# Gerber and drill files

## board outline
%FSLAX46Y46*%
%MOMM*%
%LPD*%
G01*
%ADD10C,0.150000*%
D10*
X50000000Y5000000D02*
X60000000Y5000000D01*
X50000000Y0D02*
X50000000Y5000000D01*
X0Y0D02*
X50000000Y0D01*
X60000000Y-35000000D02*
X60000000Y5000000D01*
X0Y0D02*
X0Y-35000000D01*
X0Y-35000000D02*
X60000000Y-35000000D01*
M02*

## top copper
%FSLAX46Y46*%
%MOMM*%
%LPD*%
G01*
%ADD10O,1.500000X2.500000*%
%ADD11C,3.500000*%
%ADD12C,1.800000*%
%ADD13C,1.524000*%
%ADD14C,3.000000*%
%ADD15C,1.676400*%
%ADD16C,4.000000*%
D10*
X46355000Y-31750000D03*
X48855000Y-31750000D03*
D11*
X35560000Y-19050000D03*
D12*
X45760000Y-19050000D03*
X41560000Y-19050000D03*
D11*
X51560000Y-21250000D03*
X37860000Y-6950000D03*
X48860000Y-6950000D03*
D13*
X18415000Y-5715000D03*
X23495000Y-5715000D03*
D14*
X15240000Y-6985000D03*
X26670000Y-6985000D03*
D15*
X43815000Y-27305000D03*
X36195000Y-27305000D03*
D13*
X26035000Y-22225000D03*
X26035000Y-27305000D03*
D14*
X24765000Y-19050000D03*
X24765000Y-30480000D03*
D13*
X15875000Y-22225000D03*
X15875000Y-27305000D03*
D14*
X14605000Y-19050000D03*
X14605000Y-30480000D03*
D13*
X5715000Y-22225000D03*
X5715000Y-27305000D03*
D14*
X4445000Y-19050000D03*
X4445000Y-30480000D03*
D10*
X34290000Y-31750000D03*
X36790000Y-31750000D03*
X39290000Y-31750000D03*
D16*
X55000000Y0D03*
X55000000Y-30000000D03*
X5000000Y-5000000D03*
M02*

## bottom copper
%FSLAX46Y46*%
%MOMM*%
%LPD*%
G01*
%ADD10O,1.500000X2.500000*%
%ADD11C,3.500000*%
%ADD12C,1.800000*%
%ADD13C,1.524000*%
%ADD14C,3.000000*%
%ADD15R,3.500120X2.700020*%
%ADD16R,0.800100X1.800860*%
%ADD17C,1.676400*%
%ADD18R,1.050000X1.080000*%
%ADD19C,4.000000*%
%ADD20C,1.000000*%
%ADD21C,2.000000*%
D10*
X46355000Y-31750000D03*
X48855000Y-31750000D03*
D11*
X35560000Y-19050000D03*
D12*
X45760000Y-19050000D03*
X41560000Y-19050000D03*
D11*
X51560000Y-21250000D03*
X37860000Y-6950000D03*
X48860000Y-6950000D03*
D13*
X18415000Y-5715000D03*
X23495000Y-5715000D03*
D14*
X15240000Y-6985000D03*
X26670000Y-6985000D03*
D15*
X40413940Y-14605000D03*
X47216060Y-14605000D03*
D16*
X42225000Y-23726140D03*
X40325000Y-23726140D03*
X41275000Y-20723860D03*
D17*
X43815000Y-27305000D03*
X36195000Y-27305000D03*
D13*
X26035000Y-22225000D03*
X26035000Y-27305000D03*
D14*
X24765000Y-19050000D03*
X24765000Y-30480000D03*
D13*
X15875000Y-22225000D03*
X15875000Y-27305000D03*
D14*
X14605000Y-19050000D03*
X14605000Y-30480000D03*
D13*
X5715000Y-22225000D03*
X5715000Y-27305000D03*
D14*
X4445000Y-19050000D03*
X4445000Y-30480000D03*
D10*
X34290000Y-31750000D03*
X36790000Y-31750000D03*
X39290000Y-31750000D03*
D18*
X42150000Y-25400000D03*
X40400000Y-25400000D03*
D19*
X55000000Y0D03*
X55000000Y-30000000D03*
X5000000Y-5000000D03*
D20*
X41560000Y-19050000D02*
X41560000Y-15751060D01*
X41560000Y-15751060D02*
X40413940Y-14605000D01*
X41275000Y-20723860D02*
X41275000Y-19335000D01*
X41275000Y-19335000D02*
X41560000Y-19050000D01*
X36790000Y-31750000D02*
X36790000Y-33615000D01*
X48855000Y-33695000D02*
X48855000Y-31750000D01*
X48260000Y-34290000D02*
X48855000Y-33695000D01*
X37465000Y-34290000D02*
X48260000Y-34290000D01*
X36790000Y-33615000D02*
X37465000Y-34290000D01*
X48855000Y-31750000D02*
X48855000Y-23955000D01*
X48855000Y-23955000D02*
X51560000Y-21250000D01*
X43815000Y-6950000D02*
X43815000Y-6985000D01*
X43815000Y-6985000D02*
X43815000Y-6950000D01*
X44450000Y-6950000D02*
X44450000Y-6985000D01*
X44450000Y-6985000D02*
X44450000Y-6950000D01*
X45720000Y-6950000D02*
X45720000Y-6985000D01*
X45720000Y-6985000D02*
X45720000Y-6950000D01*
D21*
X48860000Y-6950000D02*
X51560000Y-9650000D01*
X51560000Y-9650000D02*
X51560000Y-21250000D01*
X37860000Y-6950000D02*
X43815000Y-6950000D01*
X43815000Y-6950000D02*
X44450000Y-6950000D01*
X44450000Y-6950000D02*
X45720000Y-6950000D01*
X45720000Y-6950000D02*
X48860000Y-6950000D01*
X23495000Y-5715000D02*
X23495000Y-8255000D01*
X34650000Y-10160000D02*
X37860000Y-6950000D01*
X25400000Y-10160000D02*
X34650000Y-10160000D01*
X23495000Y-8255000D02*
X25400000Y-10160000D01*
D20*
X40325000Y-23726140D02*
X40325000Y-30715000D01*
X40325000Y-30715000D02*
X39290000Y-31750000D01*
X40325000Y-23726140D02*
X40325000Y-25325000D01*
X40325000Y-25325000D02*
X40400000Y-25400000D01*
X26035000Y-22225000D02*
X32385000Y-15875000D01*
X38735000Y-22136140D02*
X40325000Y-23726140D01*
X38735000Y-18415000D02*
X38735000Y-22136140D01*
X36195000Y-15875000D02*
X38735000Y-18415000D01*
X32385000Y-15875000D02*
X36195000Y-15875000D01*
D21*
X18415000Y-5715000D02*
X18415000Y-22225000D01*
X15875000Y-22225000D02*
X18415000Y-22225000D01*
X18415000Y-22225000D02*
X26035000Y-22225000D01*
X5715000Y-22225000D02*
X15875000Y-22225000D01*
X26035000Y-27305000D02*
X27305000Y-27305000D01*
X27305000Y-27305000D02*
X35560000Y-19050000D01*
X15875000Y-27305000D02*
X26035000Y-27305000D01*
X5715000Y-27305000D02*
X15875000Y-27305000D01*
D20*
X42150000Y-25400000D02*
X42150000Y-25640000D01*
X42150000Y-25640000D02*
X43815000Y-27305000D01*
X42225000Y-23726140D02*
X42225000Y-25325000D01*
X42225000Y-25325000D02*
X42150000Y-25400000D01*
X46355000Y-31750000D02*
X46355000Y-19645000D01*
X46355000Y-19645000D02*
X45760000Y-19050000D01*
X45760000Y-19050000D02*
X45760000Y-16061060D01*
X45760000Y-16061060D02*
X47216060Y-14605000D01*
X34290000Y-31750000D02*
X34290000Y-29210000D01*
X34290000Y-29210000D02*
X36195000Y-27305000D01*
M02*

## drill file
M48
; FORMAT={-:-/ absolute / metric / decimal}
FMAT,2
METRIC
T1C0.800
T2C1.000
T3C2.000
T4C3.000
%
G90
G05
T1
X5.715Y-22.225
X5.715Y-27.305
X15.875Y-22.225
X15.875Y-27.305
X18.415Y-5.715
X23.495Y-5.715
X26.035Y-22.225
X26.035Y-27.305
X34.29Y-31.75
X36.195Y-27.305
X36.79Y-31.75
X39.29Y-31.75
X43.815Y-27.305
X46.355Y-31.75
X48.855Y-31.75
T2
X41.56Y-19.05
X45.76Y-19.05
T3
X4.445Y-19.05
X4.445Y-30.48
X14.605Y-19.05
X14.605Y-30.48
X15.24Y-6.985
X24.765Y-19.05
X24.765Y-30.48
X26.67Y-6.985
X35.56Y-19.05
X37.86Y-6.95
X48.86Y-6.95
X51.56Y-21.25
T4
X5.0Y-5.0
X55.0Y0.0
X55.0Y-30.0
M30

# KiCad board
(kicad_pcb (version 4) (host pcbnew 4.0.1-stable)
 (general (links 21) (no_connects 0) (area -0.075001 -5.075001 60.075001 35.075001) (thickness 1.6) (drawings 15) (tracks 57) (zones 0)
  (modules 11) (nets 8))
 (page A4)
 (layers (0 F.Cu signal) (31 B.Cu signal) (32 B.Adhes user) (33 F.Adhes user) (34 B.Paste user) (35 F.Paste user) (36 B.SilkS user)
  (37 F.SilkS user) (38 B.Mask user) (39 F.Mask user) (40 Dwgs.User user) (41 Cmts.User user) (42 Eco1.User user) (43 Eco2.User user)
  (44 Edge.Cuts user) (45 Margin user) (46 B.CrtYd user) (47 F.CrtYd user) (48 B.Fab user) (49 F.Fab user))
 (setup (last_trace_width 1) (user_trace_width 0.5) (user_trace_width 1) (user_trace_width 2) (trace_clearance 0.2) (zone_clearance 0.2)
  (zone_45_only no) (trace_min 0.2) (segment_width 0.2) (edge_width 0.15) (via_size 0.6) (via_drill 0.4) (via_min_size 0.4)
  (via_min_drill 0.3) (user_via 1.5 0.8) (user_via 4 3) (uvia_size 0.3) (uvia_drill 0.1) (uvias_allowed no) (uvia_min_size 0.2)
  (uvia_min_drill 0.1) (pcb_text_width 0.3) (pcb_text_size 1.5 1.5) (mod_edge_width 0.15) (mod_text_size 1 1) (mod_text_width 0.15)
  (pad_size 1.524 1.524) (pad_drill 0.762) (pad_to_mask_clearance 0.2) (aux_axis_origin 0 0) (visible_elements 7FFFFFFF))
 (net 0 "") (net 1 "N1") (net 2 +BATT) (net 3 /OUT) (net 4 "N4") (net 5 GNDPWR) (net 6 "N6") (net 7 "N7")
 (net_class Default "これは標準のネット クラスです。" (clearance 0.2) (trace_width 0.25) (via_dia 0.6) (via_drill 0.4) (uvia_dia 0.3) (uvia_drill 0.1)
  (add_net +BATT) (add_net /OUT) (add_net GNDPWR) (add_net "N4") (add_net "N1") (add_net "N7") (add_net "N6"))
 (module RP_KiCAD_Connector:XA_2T (layer F.Cu) (at 46.355 31.75)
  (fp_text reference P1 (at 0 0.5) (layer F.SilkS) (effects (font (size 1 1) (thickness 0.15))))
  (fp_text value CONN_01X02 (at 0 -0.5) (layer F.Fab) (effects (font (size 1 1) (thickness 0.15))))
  (pad 2 thru_hole oval (at 0 0) (size 1.5 2.5) (drill 0.8) (layers *.Cu *.Mask F.SilkS) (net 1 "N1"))
  (pad 1 thru_hole oval (at 2.5 0) (size 1.5 2.5) (drill 0.8) (layers *.Cu *.Mask F.SilkS) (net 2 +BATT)))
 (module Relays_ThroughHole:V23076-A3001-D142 (layer F.Cu) (at 35.56 19.05 180)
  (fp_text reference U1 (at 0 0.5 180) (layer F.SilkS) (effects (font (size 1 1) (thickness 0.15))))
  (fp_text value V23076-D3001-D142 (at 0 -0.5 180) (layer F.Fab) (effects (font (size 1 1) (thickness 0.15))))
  (pad 5 thru_hole circle (at 0 0 180) (size 3.5 3.5) (drill 2) (layers *.Cu *.Mask F.SilkS) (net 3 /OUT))
  (pad 2 thru_hole circle (at -10.2 0 180) (size 1.8 1.8) (drill 1) (layers *.Cu *.Mask F.SilkS) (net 1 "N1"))
  (pad 1 thru_hole circle (at -6 0 180) (size 1.8 1.8) (drill 1) (layers *.Cu *.Mask F.SilkS) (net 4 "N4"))
  (pad 4 thru_hole circle (at -16 -2.2 180) (size 3.5 3.5) (drill 2) (layers *.Cu *.Mask F.SilkS) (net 2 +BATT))
  (pad 4 thru_hole circle (at -2.3 12.1 180) (size 3.5 3.5) (drill 2) (layers *.Cu *.Mask F.SilkS) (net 2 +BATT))
  (pad 4 thru_hole circle (at -13.3 12.1 180) (size 3.5 3.5) (drill 2) (layers *.Cu *.Mask F.SilkS) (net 2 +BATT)))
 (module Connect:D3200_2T (layer F.Cu) (at 18.415 5.715)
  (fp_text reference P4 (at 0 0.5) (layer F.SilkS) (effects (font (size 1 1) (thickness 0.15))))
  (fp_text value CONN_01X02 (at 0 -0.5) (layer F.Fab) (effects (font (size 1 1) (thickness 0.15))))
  (pad 1 thru_hole circle (at 0 0) (size 1.524 1.524) (drill 0.8) (layers *.Cu *.Mask F.SilkS) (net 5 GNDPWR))
  (pad 2 thru_hole circle (at 5.08 0) (size 1.524 1.524) (drill 0.8) (layers *.Cu *.Mask F.SilkS) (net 2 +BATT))
  (pad 3 thru_hole circle (at -3.175 1.27) (size 3 3) (drill 2) (layers *.Cu *.Mask F.SilkS))
  (pad 5 thru_hole circle (at 8.255 1.27) (size 3 3) (drill 2) (layers *.Cu *.Mask F.SilkS)))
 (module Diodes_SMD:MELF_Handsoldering (layer B.Cu) (at 43.815 14.605)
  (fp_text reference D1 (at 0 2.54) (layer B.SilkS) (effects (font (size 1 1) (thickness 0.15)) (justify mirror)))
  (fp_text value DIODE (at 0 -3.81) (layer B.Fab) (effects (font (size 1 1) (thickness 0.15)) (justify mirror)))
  (pad 1 smd rect (at -3.40106 0) (size 3.50012 2.70002) (layers B.Cu B.Paste B.Mask) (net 4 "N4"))
  (pad 2 smd rect (at 3.40106 0) (size 3.50012 2.70002) (layers B.Cu B.Paste B.Mask) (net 1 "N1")))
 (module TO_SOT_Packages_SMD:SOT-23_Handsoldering (layer B.Cu) (at 41.275 22.225 180)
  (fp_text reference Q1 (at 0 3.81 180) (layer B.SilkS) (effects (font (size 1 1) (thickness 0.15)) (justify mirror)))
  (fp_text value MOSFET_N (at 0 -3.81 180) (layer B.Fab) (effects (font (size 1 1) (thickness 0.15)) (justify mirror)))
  (pad G smd rect (at -0.95 -1.50114 180) (size 0.8001 1.80086) (layers B.Cu B.Paste B.Mask) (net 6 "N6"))
  (pad S smd rect (at 0.95 -1.50114 180) (size 0.8001 1.80086) (layers B.Cu B.Paste B.Mask) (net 5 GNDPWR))
  (pad D smd rect (at 0 1.50114 180) (size 0.8001 1.80086) (layers B.Cu B.Paste B.Mask) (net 4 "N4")))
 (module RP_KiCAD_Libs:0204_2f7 (layer F.Cu) (at 40.005 27.305 180)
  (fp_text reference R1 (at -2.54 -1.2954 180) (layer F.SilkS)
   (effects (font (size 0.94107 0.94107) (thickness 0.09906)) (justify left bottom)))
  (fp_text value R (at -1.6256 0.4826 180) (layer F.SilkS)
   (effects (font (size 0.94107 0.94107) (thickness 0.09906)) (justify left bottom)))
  (pad 1 thru_hole circle (at -3.81 0 180) (size 1.6764 1.6764) (drill 0.8) (layers *.Cu *.Mask) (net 6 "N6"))
  (pad 2 thru_hole circle (at 3.81 0 180) (size 1.6764 1.6764) (drill 0.8) (layers *.Cu *.Mask) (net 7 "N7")))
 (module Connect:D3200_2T (layer F.Cu) (at 26.035 22.225 270)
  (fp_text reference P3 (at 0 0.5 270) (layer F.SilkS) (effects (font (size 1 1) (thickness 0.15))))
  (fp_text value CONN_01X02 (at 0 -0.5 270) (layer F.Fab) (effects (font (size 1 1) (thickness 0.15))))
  (pad 1 thru_hole circle (at 0 0 270) (size 1.524 1.524) (drill 0.8) (layers *.Cu *.Mask F.SilkS) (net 5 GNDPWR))
  (pad 2 thru_hole circle (at 5.08 0 270) (size 1.524 1.524) (drill 0.8) (layers *.Cu *.Mask F.SilkS) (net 3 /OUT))
  (pad 3 thru_hole circle (at -3.175 1.27 270) (size 3 3) (drill 2) (layers *.Cu *.Mask F.SilkS))
  (pad 5 thru_hole circle (at 8.255 1.27 270) (size 3 3) (drill 2) (layers *.Cu *.Mask F.SilkS)))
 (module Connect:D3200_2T (layer F.Cu) (at 15.875 22.225 270)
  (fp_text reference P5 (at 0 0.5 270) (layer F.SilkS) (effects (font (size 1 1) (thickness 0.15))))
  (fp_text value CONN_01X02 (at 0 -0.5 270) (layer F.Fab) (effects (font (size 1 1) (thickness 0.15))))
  (pad 1 thru_hole circle (at 0 0 270) (size 1.524 1.524) (drill 0.8) (layers *.Cu *.Mask F.SilkS) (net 5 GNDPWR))
  (pad 2 thru_hole circle (at 5.08 0 270) (size 1.524 1.524) (drill 0.8) (layers *.Cu *.Mask F.SilkS) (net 3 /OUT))
  (pad 3 thru_hole circle (at -3.175 1.27 270) (size 3 3) (drill 2) (layers *.Cu *.Mask F.SilkS))
  (pad 5 thru_hole circle (at 8.255 1.27 270) (size 3 3) (drill 2) (layers *.Cu *.Mask F.SilkS)))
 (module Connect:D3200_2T (layer F.Cu) (at 5.715 22.225 270)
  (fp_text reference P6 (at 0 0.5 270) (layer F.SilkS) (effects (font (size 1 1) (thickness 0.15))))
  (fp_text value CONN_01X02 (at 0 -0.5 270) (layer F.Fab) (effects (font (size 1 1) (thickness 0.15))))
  (pad 1 thru_hole circle (at 0 0 270) (size 1.524 1.524) (drill 0.8) (layers *.Cu *.Mask F.SilkS) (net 5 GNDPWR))
  (pad 2 thru_hole circle (at 5.08 0 270) (size 1.524 1.524) (drill 0.8) (layers *.Cu *.Mask F.SilkS) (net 3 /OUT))
  (pad 3 thru_hole circle (at -3.175 1.27 270) (size 3 3) (drill 2) (layers *.Cu *.Mask F.SilkS))
  (pad 5 thru_hole circle (at 8.255 1.27 270) (size 3 3) (drill 2) (layers *.Cu *.Mask F.SilkS)))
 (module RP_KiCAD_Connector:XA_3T (layer F.Cu) (at 34.29 31.75)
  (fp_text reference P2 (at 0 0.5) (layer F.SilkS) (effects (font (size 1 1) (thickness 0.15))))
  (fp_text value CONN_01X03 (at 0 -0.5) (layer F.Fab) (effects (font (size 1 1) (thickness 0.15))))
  (pad 3 thru_hole oval (at 0 0) (size 1.5 2.5) (drill 0.8) (layers *.Cu *.Mask F.SilkS) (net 7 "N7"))
  (pad 2 thru_hole oval (at 2.5 0) (size 1.5 2.5) (drill 0.8) (layers *.Cu *.Mask F.SilkS) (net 2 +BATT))
  (pad 1 thru_hole oval (at 5 0) (size 1.5 2.5) (drill 0.8) (layers *.Cu *.Mask F.SilkS) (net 5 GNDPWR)))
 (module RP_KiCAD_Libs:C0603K (layer B.Cu) (at 41.275 25.4 180)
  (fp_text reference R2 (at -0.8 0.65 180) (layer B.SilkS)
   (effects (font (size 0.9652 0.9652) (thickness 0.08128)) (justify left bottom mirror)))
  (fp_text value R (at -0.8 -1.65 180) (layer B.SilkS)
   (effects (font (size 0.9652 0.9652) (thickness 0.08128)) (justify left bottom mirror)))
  (pad 1 smd rect (at -0.875 0 180) (size 1.05 1.08) (layers B.Cu B.Paste B.Mask) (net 6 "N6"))
  (pad 2 smd rect (at 0.875 0 180) (size 1.05 1.08) (layers B.Cu B.Paste B.Mask) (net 5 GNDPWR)))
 (gr_line (start 50 -5) (end 60 -5) (angle 90) (layer Edge.Cuts) (width 0.15))
 (gr_line (start 50 0) (end 50 -5) (angle 90) (layer Edge.Cuts) (width 0.15))
 (gr_line (start 0 0) (end 50 0) (angle 90) (layer Edge.Cuts) (width 0.15))
 (gr_line (start 60 35) (end 60 -5) (angle 90) (layer Edge.Cuts) (width 0.15))
 (gr_line (start 0 0) (end 0 35) (angle 90) (layer Edge.Cuts) (width 0.15))
 (gr_line (start 0 35) (end 60 35) (angle 90) (layer Edge.Cuts) (width 0.15))
 (via (at 55 0) (size 4) (drill 3) (layers F.Cu B.Cu) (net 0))
 (via (at 55 30) (size 4) (drill 3) (layers F.Cu B.Cu) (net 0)) (via (at 5 5) (size 4) (drill 3) (layers F.Cu B.Cu) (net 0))
 (segment (start 41.56 19.05) (end 41.56 15.75106) (width 1) (layer B.Cu) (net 4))
 (segment (start 41.56 15.75106) (end 40.41394 14.605) (width 1) (layer B.Cu) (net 4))
 (segment (start 41.275 20.72386) (end 41.275 19.335) (width 1) (layer B.Cu) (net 4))
 (segment (start 41.275 19.335) (end 41.56 19.05) (width 1) (layer B.Cu) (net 4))
 (segment (start 36.79 31.75) (end 36.79 33.615) (width 1) (layer B.Cu) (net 2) (status 400000))
 (segment (start 48.855 33.695) (end 48.855 31.75) (width 1) (layer B.Cu) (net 2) (status 800000))
 (segment (start 48.26 34.29) (end 48.855 33.695) (width 1) (layer B.Cu) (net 2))
 (segment (start 37.465 34.29) (end 48.26 34.29) (width 1) (layer B.Cu) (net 2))
 (segment (start 36.79 33.615) (end 37.465 34.29) (width 1) (layer B.Cu) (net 2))
 (segment (start 48.855 31.75) (end 48.855 23.955) (width 1) (layer B.Cu) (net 2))
 (segment (start 48.855 23.955) (end 51.56 21.25) (width 1) (layer B.Cu) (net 2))
 (segment (start 43.815 6.95) (end 43.815 6.985) (width 1) (layer B.Cu) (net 2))
 (segment (start 43.815 6.985) (end 43.815 6.95) (width 1) (layer B.Cu) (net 2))
 (segment (start 44.45 6.95) (end 44.45 6.985) (width 1) (layer B.Cu) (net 2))
 (segment (start 44.45 6.985) (end 44.45 6.95) (width 1) (layer B.Cu) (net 2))
 (segment (start 45.72 6.95) (end 45.72 6.985) (width 1) (layer B.Cu) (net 2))
 (segment (start 45.72 6.985) (end 45.72 6.95) (width 1) (layer B.Cu) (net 2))
 (segment (start 48.86 6.95) (end 51.56 9.65) (width 2) (layer B.Cu) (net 2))
 (segment (start 51.56 9.65) (end 51.56 21.25) (width 2) (layer B.Cu) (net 2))
 (segment (start 37.86 6.95) (end 43.815 6.95) (width 2) (layer B.Cu) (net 2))
 (segment (start 43.815 6.95) (end 44.45 6.95) (width 2) (layer B.Cu) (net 2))
 (segment (start 44.45 6.95) (end 45.72 6.95) (width 2) (layer B.Cu) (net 2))
 (segment (start 45.72 6.95) (end 48.86 6.95) (width 2) (layer B.Cu) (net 2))
 (segment (start 23.495 5.715) (end 23.495 8.255) (width 2) (layer B.Cu) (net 2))
 (segment (start 34.65 10.16) (end 37.86 6.95) (width 2) (layer B.Cu) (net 2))
 (segment (start 25.4 10.16) (end 34.65 10.16) (width 2) (layer B.Cu) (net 2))
 (segment (start 23.495 8.255) (end 25.4 10.16) (width 2) (layer B.Cu) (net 2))
 (segment (start 40.325 23.72614) (end 40.325 30.715) (width 1) (layer B.Cu) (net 5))
 (segment (start 40.325 30.715) (end 39.29 31.75) (width 1) (layer B.Cu) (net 5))
 (segment (start 40.325 23.72614) (end 40.325 25.325) (width 1) (layer B.Cu) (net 5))
 (segment (start 40.325 25.325) (end 40.4 25.4) (width 1) (layer B.Cu) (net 5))
 (segment (start 26.035 22.225) (end 32.385 15.875) (width 1) (layer B.Cu) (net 5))
 (segment (start 38.735 22.13614) (end 40.325 23.72614) (width 1) (layer B.Cu) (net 5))
 (segment (start 38.735 18.415) (end 38.735 22.13614) (width 1) (layer B.Cu) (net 5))
 (segment (start 36.195 15.875) (end 38.735 18.415) (width 1) (layer B.Cu) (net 5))
 (segment (start 32.385 15.875) (end 36.195 15.875) (width 1) (layer B.Cu) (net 5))
 (segment (start 18.415 5.715) (end 18.415 22.225) (width 2) (layer B.Cu) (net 5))
 (segment (start 15.875 22.225) (end 18.415 22.225) (width 2) (layer B.Cu) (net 5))
 (segment (start 18.415 22.225) (end 26.035 22.225) (width 2) (layer B.Cu) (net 5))
 (segment (start 5.715 22.225) (end 15.875 22.225) (width 2) (layer B.Cu) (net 5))
 (segment (start 26.035 27.305) (end 27.305 27.305) (width 2) (layer B.Cu) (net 3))
 (segment (start 27.305 27.305) (end 35.56 19.05) (width 2) (layer B.Cu) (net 3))
 (segment (start 15.875 27.305) (end 26.035 27.305) (width 2) (layer B.Cu) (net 3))
 (segment (start 5.715 27.305) (end 15.875 27.305) (width 2) (layer B.Cu) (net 3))
 (segment (start 42.15 25.4) (end 42.15 25.64) (width 1) (layer B.Cu) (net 6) (status C00000))
 (segment (start 42.15 25.64) (end 43.815 27.305) (width 1) (layer B.Cu) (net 6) (status C00000))
 (segment (start 42.225 23.72614) (end 42.225 25.325) (width 1) (layer B.Cu) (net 6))
 (segment (start 42.225 25.325) (end 42.15 25.4) (width 1) (layer B.Cu) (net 6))
 (segment (start 46.355 31.75) (end 46.355 19.645) (width 1) (layer B.Cu) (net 1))
 (segment (start 46.355 19.645) (end 45.76 19.05) (width 1) (layer B.Cu) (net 1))
 (segment (start 45.76 19.05) (end 45.76 16.06106) (width 1) (layer B.Cu) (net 1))
 (segment (start 45.76 16.06106) (end 47.21606 14.605) (width 1) (layer B.Cu) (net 1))
 (segment (start 34.29 31.75) (end 34.29 29.21) (width 1) (layer B.Cu) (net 7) (status 400000))
 (segment (start 34.29 29.21) (end 36.195 27.305) (width 1) (layer B.Cu) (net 7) (status 800000)))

